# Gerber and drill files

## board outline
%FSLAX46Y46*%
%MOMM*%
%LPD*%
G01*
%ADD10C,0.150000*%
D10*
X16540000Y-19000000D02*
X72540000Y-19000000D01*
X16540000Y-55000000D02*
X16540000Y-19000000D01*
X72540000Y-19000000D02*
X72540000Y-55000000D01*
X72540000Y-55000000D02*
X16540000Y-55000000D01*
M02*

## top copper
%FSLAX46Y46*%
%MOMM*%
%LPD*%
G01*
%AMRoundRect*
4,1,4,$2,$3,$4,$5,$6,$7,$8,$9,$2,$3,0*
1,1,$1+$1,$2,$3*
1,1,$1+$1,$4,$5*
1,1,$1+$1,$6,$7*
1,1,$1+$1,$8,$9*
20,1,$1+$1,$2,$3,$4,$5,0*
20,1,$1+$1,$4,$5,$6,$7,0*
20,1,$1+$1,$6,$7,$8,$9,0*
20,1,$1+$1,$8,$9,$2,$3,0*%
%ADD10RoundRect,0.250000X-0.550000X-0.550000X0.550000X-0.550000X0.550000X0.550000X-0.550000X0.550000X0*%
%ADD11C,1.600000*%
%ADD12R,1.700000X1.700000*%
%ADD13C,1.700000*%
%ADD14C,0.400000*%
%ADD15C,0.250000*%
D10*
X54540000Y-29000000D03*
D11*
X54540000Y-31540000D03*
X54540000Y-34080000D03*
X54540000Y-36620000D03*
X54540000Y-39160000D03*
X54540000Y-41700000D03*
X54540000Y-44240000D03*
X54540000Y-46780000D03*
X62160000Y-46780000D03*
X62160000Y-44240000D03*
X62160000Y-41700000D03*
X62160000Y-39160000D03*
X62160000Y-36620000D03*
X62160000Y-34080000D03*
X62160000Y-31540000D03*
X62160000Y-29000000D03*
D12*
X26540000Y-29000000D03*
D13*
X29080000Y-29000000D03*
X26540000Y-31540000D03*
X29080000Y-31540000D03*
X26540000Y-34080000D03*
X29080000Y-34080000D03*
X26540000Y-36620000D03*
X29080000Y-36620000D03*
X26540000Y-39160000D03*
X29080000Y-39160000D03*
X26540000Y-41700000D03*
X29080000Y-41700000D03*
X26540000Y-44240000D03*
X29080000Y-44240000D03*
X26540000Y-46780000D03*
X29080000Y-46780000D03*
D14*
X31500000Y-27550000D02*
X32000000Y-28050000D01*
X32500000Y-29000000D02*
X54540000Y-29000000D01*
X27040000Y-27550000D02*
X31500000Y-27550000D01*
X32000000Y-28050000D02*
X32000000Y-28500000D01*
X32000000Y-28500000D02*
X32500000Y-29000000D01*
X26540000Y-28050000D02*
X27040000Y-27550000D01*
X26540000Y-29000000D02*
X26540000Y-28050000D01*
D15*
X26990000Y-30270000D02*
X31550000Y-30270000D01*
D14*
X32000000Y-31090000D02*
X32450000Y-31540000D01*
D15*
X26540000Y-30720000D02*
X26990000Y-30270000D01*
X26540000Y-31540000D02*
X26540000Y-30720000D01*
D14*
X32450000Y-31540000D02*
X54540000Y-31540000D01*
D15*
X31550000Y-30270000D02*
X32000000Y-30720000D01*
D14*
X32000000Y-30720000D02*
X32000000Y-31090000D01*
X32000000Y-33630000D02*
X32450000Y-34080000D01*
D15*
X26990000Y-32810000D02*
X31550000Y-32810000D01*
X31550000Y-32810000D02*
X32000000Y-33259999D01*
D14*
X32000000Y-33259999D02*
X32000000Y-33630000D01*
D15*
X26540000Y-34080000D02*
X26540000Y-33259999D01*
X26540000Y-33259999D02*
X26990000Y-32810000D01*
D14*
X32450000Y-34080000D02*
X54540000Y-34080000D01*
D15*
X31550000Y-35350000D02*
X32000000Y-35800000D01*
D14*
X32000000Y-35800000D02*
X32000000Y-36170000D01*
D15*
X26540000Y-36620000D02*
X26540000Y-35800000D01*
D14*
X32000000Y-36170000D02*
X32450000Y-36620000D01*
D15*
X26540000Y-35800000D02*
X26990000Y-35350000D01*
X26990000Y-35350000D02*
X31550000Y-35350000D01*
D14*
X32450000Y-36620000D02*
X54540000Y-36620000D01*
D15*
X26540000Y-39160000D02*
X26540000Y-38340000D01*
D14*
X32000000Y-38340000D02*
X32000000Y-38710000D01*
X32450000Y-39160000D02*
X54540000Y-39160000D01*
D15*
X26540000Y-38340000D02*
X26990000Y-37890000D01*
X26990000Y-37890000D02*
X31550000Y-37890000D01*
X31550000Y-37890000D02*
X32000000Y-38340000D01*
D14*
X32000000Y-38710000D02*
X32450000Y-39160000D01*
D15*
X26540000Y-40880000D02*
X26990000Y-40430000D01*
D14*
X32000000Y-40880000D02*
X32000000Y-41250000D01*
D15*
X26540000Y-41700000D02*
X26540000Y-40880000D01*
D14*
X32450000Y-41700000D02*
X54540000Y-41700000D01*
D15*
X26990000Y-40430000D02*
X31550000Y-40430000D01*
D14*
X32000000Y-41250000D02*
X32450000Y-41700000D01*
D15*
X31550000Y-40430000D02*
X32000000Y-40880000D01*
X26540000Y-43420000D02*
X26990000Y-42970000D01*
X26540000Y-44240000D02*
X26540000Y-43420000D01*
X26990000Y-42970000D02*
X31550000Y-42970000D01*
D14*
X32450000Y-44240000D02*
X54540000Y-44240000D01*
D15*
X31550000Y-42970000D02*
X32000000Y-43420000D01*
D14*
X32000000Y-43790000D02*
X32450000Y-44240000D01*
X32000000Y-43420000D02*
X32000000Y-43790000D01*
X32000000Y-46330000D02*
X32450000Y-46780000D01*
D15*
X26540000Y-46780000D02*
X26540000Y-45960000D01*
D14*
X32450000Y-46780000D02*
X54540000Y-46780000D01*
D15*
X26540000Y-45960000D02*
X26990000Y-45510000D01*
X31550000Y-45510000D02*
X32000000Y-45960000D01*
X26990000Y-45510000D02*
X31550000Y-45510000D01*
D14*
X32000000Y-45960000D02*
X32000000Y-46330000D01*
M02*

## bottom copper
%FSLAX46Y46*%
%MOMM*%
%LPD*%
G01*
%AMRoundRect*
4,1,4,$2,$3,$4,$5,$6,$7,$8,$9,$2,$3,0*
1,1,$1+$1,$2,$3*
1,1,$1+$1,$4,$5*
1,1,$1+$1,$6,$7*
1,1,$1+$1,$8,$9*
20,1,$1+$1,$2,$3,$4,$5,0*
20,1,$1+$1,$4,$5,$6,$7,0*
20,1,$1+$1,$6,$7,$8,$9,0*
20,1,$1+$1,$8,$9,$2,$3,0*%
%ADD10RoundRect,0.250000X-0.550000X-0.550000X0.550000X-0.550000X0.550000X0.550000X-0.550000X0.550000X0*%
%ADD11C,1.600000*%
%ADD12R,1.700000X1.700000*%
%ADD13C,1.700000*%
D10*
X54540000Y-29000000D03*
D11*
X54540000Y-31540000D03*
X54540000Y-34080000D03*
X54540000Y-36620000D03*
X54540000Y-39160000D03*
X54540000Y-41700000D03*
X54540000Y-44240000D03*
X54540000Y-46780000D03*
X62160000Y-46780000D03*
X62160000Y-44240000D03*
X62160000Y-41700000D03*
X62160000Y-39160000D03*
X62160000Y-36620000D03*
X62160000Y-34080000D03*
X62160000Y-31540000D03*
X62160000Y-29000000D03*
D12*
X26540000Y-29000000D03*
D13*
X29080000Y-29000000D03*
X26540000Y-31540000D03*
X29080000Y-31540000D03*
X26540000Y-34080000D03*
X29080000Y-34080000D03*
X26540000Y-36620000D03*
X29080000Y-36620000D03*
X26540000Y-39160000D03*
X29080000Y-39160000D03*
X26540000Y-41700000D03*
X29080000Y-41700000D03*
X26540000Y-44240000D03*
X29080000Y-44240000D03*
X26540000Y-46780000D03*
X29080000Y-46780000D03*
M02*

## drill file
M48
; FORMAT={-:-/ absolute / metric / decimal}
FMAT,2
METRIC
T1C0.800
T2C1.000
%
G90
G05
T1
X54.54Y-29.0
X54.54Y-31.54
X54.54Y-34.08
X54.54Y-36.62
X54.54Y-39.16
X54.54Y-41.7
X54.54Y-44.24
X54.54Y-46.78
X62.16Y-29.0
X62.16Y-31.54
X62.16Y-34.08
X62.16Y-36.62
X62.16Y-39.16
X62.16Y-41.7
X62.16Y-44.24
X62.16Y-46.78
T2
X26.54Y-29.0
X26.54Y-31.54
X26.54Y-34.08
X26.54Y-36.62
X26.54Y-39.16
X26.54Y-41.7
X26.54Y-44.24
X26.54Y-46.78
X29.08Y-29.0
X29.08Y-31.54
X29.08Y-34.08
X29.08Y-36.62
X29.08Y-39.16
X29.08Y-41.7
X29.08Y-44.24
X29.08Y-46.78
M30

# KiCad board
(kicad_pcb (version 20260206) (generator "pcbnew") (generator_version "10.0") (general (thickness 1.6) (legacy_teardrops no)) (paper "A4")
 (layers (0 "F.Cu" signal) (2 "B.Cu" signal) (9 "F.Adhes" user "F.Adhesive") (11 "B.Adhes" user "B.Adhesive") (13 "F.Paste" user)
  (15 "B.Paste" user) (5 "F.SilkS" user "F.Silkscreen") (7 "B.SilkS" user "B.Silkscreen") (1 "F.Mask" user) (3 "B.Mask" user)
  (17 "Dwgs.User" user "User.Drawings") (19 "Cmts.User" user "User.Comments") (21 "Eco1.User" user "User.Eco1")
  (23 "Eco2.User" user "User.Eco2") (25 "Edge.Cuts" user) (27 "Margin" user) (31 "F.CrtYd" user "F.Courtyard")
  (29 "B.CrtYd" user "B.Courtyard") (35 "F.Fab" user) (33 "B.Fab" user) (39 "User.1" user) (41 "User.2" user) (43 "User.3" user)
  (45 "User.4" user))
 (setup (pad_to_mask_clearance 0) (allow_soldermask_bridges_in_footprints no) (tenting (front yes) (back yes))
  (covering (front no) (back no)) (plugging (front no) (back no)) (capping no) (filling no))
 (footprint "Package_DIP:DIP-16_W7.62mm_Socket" (layer "F.Cu") (at 54.54 29)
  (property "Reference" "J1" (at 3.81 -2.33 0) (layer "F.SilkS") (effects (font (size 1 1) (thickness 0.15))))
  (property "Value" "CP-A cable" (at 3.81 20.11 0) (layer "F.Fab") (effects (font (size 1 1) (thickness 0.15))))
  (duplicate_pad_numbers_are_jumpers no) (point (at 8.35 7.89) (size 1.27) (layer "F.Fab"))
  (pad "1" thru_hole roundrect (at 0 0) (size 1.6 1.6) (drill 0.8) (layers "*.Cu" "*.Mask") (remove_unused_layers no)
   (roundrect_rratio 0.15625) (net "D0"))
  (pad "2" thru_hole circle (at 0 2.54) (size 1.6 1.6) (drill 0.8) (layers "*.Cu" "*.Mask") (remove_unused_layers no) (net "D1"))
  (pad "3" thru_hole circle (at 0 5.08) (size 1.6 1.6) (drill 0.8) (layers "*.Cu" "*.Mask") (remove_unused_layers no) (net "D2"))
  (pad "4" thru_hole circle (at 0 7.62) (size 1.6 1.6) (drill 0.8) (layers "*.Cu" "*.Mask") (remove_unused_layers no) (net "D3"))
  (pad "5" thru_hole circle (at 0 10.16) (size 1.6 1.6) (drill 0.8) (layers "*.Cu" "*.Mask") (remove_unused_layers no) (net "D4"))
  (pad "6" thru_hole circle (at 0 12.7) (size 1.6 1.6) (drill 0.8) (layers "*.Cu" "*.Mask") (remove_unused_layers no) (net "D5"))
  (pad "7" thru_hole circle (at 0 15.24) (size 1.6 1.6) (drill 0.8) (layers "*.Cu" "*.Mask") (remove_unused_layers no) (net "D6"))
  (pad "8" thru_hole circle (at 0 17.78) (size 1.6 1.6) (drill 0.8) (layers "*.Cu" "*.Mask") (remove_unused_layers no) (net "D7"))
  (pad "9" thru_hole circle (at 7.62 17.78) (size 1.6 1.6) (drill 0.8) (layers "*.Cu" "*.Mask") (remove_unused_layers no))
  (pad "10" thru_hole circle (at 7.62 15.24) (size 1.6 1.6) (drill 0.8) (layers "*.Cu" "*.Mask") (remove_unused_layers no))
  (pad "11" thru_hole circle (at 7.62 12.7) (size 1.6 1.6) (drill 0.8) (layers "*.Cu" "*.Mask") (remove_unused_layers no))
  (pad "12" thru_hole circle (at 7.62 10.16) (size 1.6 1.6) (drill 0.8) (layers "*.Cu" "*.Mask") (remove_unused_layers no))
  (pad "13" thru_hole circle (at 7.62 7.62) (size 1.6 1.6) (drill 0.8) (layers "*.Cu" "*.Mask") (remove_unused_layers no))
  (pad "14" thru_hole circle (at 7.62 5.08) (size 1.6 1.6) (drill 0.8) (layers "*.Cu" "*.Mask") (remove_unused_layers no))
  (pad "15" thru_hole circle (at 7.62 2.54) (size 1.6 1.6) (drill 0.8) (layers "*.Cu" "*.Mask") (remove_unused_layers no))
  (pad "16" thru_hole circle (at 7.62 0) (size 1.6 1.6) (drill 0.8) (layers "*.Cu" "*.Mask") (remove_unused_layers no)))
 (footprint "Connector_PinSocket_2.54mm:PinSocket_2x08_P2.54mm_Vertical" (layer "B.Cu") (at 26.54 29 180)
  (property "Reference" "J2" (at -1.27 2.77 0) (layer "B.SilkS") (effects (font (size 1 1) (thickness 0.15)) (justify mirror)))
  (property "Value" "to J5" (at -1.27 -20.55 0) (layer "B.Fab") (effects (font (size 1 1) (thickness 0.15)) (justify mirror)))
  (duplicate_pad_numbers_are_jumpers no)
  (pad "1" thru_hole rect (at 0 0 180) (size 1.7 1.7) (drill 1) (layers "*.Cu" "*.Mask") (remove_unused_layers no) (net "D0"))
  (pad "2" thru_hole circle (at -2.54 0 180) (size 1.7 1.7) (drill 1) (layers "*.Cu" "*.Mask") (remove_unused_layers no))
  (pad "3" thru_hole circle (at 0 -2.54 180) (size 1.7 1.7) (drill 1) (layers "*.Cu" "*.Mask") (remove_unused_layers no) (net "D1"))
  (pad "4" thru_hole circle (at -2.54 -2.54 180) (size 1.7 1.7) (drill 1) (layers "*.Cu" "*.Mask") (remove_unused_layers no))
  (pad "5" thru_hole circle (at 0 -5.08 180) (size 1.7 1.7) (drill 1) (layers "*.Cu" "*.Mask") (remove_unused_layers no) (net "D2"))
  (pad "6" thru_hole circle (at -2.54 -5.08 180) (size 1.7 1.7) (drill 1) (layers "*.Cu" "*.Mask") (remove_unused_layers no))
  (pad "7" thru_hole circle (at 0 -7.62 180) (size 1.7 1.7) (drill 1) (layers "*.Cu" "*.Mask") (remove_unused_layers no) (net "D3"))
  (pad "8" thru_hole circle (at -2.54 -7.62 180) (size 1.7 1.7) (drill 1) (layers "*.Cu" "*.Mask") (remove_unused_layers no))
  (pad "9" thru_hole circle (at 0 -10.16 180) (size 1.7 1.7) (drill 1) (layers "*.Cu" "*.Mask") (remove_unused_layers no) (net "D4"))
  (pad "10" thru_hole circle (at -2.54 -10.16 180) (size 1.7 1.7) (drill 1) (layers "*.Cu" "*.Mask") (remove_unused_layers no))
  (pad "11" thru_hole circle (at 0 -12.7 180) (size 1.7 1.7) (drill 1) (layers "*.Cu" "*.Mask") (remove_unused_layers no) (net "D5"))
  (pad "12" thru_hole circle (at -2.54 -12.7 180) (size 1.7 1.7) (drill 1) (layers "*.Cu" "*.Mask") (remove_unused_layers no))
  (pad "13" thru_hole circle (at 0 -15.24 180) (size 1.7 1.7) (drill 1) (layers "*.Cu" "*.Mask") (remove_unused_layers no) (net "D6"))
  (pad "14" thru_hole circle (at -2.54 -15.24 180) (size 1.7 1.7) (drill 1) (layers "*.Cu" "*.Mask") (remove_unused_layers no))
  (pad "15" thru_hole circle (at 0 -17.78 180) (size 1.7 1.7) (drill 1) (layers "*.Cu" "*.Mask") (remove_unused_layers no) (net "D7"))
  (pad "16" thru_hole circle (at -2.54 -17.78 180) (size 1.7 1.7) (drill 1) (layers "*.Cu" "*.Mask") (remove_unused_layers no)))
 (gr_line (start 16.54 19) (end 72.54 19) (stroke (width 0.15) (type solid)) (layer "Edge.Cuts"))
 (gr_line (start 16.54 55) (end 16.54 19) (stroke (width 0.15) (type solid)) (layer "Edge.Cuts"))
 (gr_line (start 72.54 19) (end 72.54 55) (stroke (width 0.15) (type solid)) (layer "Edge.Cuts"))
 (gr_line (start 72.54 55) (end 16.54 55) (stroke (width 0.15) (type solid)) (layer "Edge.Cuts"))
 (segment (start 31.5 27.55) (end 32 28.05) (width 0.4) (layer "F.Cu") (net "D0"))
 (segment (start 32.5 29) (end 54.54 29) (width 0.4) (layer "F.Cu") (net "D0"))
 (segment (start 27.04 27.55) (end 31.5 27.55) (width 0.4) (layer "F.Cu") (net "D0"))
 (segment (start 32 28.05) (end 32 28.5) (width 0.4) (layer "F.Cu") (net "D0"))
 (segment (start 32 28.5) (end 32.5 29) (width 0.4) (layer "F.Cu") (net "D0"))
 (segment (start 26.54 28.05) (end 27.04 27.55) (width 0.4) (layer "F.Cu") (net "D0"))
 (segment (start 26.54 29) (end 26.54 28.05) (width 0.4) (layer "F.Cu") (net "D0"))
 (segment (start 26.99 30.27) (end 31.55 30.27) (width 0.25) (layer "F.Cu") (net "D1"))
 (segment (start 32 31.09) (end 32.45 31.54) (width 0.4) (layer "F.Cu") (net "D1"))
 (segment (start 26.54 30.72) (end 26.99 30.27) (width 0.25) (layer "F.Cu") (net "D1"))
 (segment (start 26.54 31.54) (end 26.54 30.72) (width 0.25) (layer "F.Cu") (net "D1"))
 (segment (start 32.45 31.54) (end 54.54 31.54) (width 0.4) (layer "F.Cu") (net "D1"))
 (segment (start 31.55 30.27) (end 32 30.72) (width 0.25) (layer "F.Cu") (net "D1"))
 (segment (start 32 30.72) (end 32 31.09) (width 0.4) (layer "F.Cu") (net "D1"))
 (segment (start 32 33.63) (end 32.45 34.08) (width 0.4) (layer "F.Cu") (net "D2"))
 (segment (start 26.99 32.81) (end 31.55 32.81) (width 0.25) (layer "F.Cu") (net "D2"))
 (segment (start 31.55 32.81) (end 32 33.259999) (width 0.25) (layer "F.Cu") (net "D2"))
 (segment (start 32 33.259999) (end 32 33.63) (width 0.4) (layer "F.Cu") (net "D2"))
 (segment (start 26.54 34.08) (end 26.54 33.259999) (width 0.25) (layer "F.Cu") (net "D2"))
 (segment (start 26.54 33.259999) (end 26.99 32.81) (width 0.25) (layer "F.Cu") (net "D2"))
 (segment (start 32.45 34.08) (end 54.54 34.08) (width 0.4) (layer "F.Cu") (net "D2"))
 (segment (start 31.55 35.35) (end 32 35.8) (width 0.25) (layer "F.Cu") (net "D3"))
 (segment (start 32 35.8) (end 32 36.17) (width 0.4) (layer "F.Cu") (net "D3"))
 (segment (start 26.54 36.62) (end 26.54 35.8) (width 0.25) (layer "F.Cu") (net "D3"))
 (segment (start 32 36.17) (end 32.45 36.62) (width 0.4) (layer "F.Cu") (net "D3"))
 (segment (start 26.54 35.8) (end 26.99 35.35) (width 0.25) (layer "F.Cu") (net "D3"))
 (segment (start 26.99 35.35) (end 31.55 35.35) (width 0.25) (layer "F.Cu") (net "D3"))
 (segment (start 32.45 36.62) (end 54.54 36.62) (width 0.4) (layer "F.Cu") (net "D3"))
 (segment (start 26.54 39.16) (end 26.54 38.34) (width 0.25) (layer "F.Cu") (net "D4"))
 (segment (start 32 38.34) (end 32 38.71) (width 0.4) (layer "F.Cu") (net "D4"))
 (segment (start 32.45 39.16) (end 54.54 39.16) (width 0.4) (layer "F.Cu") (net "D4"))
 (segment (start 26.54 38.34) (end 26.99 37.89) (width 0.25) (layer "F.Cu") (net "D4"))
 (segment (start 26.99 37.89) (end 31.55 37.89) (width 0.25) (layer "F.Cu") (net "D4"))
 (segment (start 31.55 37.89) (end 32 38.34) (width 0.25) (layer "F.Cu") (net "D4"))
 (segment (start 32 38.71) (end 32.45 39.16) (width 0.4) (layer "F.Cu") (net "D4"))
 (segment (start 26.54 40.88) (end 26.99 40.43) (width 0.25) (layer "F.Cu") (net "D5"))
 (segment (start 32 40.88) (end 32 41.25) (width 0.4) (layer "F.Cu") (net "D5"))
 (segment (start 26.54 41.7) (end 26.54 40.88) (width 0.25) (layer "F.Cu") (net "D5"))
 (segment (start 32.45 41.7) (end 54.54 41.7) (width 0.4) (layer "F.Cu") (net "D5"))
 (segment (start 26.99 40.43) (end 31.55 40.43) (width 0.25) (layer "F.Cu") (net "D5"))
 (segment (start 32 41.25) (end 32.45 41.7) (width 0.4) (layer "F.Cu") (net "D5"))
 (segment (start 31.55 40.43) (end 32 40.88) (width 0.25) (layer "F.Cu") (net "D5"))
 (segment (start 26.54 43.42) (end 26.99 42.97) (width 0.25) (layer "F.Cu") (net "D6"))
 (segment (start 26.54 44.24) (end 26.54 43.42) (width 0.25) (layer "F.Cu") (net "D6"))
 (segment (start 26.99 42.97) (end 31.55 42.97) (width 0.25) (layer "F.Cu") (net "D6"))
 (segment (start 32.45 44.24) (end 54.54 44.24) (width 0.4) (layer "F.Cu") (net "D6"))
 (segment (start 31.55 42.97) (end 32 43.42) (width 0.25) (layer "F.Cu") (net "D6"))
 (segment (start 32 43.79) (end 32.45 44.24) (width 0.4) (layer "F.Cu") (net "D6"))
 (segment (start 32 43.42) (end 32 43.79) (width 0.4) (layer "F.Cu") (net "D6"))
 (segment (start 32 46.33) (end 32.45 46.78) (width 0.4) (layer "F.Cu") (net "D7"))
 (segment (start 26.54 46.78) (end 26.54 45.96) (width 0.25) (layer "F.Cu") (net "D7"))
 (segment (start 32.45 46.78) (end 54.54 46.78) (width 0.4) (layer "F.Cu") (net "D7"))
 (segment (start 26.54 45.96) (end 26.99 45.51) (width 0.25) (layer "F.Cu") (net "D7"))
 (segment (start 31.55 45.51) (end 32 45.96) (width 0.25) (layer "F.Cu") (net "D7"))
 (segment (start 26.99 45.51) (end 31.55 45.51) (width 0.25) (layer "F.Cu") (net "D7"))
 (segment (start 32 45.96) (end 32 46.33) (width 0.4) (layer "F.Cu") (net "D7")))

